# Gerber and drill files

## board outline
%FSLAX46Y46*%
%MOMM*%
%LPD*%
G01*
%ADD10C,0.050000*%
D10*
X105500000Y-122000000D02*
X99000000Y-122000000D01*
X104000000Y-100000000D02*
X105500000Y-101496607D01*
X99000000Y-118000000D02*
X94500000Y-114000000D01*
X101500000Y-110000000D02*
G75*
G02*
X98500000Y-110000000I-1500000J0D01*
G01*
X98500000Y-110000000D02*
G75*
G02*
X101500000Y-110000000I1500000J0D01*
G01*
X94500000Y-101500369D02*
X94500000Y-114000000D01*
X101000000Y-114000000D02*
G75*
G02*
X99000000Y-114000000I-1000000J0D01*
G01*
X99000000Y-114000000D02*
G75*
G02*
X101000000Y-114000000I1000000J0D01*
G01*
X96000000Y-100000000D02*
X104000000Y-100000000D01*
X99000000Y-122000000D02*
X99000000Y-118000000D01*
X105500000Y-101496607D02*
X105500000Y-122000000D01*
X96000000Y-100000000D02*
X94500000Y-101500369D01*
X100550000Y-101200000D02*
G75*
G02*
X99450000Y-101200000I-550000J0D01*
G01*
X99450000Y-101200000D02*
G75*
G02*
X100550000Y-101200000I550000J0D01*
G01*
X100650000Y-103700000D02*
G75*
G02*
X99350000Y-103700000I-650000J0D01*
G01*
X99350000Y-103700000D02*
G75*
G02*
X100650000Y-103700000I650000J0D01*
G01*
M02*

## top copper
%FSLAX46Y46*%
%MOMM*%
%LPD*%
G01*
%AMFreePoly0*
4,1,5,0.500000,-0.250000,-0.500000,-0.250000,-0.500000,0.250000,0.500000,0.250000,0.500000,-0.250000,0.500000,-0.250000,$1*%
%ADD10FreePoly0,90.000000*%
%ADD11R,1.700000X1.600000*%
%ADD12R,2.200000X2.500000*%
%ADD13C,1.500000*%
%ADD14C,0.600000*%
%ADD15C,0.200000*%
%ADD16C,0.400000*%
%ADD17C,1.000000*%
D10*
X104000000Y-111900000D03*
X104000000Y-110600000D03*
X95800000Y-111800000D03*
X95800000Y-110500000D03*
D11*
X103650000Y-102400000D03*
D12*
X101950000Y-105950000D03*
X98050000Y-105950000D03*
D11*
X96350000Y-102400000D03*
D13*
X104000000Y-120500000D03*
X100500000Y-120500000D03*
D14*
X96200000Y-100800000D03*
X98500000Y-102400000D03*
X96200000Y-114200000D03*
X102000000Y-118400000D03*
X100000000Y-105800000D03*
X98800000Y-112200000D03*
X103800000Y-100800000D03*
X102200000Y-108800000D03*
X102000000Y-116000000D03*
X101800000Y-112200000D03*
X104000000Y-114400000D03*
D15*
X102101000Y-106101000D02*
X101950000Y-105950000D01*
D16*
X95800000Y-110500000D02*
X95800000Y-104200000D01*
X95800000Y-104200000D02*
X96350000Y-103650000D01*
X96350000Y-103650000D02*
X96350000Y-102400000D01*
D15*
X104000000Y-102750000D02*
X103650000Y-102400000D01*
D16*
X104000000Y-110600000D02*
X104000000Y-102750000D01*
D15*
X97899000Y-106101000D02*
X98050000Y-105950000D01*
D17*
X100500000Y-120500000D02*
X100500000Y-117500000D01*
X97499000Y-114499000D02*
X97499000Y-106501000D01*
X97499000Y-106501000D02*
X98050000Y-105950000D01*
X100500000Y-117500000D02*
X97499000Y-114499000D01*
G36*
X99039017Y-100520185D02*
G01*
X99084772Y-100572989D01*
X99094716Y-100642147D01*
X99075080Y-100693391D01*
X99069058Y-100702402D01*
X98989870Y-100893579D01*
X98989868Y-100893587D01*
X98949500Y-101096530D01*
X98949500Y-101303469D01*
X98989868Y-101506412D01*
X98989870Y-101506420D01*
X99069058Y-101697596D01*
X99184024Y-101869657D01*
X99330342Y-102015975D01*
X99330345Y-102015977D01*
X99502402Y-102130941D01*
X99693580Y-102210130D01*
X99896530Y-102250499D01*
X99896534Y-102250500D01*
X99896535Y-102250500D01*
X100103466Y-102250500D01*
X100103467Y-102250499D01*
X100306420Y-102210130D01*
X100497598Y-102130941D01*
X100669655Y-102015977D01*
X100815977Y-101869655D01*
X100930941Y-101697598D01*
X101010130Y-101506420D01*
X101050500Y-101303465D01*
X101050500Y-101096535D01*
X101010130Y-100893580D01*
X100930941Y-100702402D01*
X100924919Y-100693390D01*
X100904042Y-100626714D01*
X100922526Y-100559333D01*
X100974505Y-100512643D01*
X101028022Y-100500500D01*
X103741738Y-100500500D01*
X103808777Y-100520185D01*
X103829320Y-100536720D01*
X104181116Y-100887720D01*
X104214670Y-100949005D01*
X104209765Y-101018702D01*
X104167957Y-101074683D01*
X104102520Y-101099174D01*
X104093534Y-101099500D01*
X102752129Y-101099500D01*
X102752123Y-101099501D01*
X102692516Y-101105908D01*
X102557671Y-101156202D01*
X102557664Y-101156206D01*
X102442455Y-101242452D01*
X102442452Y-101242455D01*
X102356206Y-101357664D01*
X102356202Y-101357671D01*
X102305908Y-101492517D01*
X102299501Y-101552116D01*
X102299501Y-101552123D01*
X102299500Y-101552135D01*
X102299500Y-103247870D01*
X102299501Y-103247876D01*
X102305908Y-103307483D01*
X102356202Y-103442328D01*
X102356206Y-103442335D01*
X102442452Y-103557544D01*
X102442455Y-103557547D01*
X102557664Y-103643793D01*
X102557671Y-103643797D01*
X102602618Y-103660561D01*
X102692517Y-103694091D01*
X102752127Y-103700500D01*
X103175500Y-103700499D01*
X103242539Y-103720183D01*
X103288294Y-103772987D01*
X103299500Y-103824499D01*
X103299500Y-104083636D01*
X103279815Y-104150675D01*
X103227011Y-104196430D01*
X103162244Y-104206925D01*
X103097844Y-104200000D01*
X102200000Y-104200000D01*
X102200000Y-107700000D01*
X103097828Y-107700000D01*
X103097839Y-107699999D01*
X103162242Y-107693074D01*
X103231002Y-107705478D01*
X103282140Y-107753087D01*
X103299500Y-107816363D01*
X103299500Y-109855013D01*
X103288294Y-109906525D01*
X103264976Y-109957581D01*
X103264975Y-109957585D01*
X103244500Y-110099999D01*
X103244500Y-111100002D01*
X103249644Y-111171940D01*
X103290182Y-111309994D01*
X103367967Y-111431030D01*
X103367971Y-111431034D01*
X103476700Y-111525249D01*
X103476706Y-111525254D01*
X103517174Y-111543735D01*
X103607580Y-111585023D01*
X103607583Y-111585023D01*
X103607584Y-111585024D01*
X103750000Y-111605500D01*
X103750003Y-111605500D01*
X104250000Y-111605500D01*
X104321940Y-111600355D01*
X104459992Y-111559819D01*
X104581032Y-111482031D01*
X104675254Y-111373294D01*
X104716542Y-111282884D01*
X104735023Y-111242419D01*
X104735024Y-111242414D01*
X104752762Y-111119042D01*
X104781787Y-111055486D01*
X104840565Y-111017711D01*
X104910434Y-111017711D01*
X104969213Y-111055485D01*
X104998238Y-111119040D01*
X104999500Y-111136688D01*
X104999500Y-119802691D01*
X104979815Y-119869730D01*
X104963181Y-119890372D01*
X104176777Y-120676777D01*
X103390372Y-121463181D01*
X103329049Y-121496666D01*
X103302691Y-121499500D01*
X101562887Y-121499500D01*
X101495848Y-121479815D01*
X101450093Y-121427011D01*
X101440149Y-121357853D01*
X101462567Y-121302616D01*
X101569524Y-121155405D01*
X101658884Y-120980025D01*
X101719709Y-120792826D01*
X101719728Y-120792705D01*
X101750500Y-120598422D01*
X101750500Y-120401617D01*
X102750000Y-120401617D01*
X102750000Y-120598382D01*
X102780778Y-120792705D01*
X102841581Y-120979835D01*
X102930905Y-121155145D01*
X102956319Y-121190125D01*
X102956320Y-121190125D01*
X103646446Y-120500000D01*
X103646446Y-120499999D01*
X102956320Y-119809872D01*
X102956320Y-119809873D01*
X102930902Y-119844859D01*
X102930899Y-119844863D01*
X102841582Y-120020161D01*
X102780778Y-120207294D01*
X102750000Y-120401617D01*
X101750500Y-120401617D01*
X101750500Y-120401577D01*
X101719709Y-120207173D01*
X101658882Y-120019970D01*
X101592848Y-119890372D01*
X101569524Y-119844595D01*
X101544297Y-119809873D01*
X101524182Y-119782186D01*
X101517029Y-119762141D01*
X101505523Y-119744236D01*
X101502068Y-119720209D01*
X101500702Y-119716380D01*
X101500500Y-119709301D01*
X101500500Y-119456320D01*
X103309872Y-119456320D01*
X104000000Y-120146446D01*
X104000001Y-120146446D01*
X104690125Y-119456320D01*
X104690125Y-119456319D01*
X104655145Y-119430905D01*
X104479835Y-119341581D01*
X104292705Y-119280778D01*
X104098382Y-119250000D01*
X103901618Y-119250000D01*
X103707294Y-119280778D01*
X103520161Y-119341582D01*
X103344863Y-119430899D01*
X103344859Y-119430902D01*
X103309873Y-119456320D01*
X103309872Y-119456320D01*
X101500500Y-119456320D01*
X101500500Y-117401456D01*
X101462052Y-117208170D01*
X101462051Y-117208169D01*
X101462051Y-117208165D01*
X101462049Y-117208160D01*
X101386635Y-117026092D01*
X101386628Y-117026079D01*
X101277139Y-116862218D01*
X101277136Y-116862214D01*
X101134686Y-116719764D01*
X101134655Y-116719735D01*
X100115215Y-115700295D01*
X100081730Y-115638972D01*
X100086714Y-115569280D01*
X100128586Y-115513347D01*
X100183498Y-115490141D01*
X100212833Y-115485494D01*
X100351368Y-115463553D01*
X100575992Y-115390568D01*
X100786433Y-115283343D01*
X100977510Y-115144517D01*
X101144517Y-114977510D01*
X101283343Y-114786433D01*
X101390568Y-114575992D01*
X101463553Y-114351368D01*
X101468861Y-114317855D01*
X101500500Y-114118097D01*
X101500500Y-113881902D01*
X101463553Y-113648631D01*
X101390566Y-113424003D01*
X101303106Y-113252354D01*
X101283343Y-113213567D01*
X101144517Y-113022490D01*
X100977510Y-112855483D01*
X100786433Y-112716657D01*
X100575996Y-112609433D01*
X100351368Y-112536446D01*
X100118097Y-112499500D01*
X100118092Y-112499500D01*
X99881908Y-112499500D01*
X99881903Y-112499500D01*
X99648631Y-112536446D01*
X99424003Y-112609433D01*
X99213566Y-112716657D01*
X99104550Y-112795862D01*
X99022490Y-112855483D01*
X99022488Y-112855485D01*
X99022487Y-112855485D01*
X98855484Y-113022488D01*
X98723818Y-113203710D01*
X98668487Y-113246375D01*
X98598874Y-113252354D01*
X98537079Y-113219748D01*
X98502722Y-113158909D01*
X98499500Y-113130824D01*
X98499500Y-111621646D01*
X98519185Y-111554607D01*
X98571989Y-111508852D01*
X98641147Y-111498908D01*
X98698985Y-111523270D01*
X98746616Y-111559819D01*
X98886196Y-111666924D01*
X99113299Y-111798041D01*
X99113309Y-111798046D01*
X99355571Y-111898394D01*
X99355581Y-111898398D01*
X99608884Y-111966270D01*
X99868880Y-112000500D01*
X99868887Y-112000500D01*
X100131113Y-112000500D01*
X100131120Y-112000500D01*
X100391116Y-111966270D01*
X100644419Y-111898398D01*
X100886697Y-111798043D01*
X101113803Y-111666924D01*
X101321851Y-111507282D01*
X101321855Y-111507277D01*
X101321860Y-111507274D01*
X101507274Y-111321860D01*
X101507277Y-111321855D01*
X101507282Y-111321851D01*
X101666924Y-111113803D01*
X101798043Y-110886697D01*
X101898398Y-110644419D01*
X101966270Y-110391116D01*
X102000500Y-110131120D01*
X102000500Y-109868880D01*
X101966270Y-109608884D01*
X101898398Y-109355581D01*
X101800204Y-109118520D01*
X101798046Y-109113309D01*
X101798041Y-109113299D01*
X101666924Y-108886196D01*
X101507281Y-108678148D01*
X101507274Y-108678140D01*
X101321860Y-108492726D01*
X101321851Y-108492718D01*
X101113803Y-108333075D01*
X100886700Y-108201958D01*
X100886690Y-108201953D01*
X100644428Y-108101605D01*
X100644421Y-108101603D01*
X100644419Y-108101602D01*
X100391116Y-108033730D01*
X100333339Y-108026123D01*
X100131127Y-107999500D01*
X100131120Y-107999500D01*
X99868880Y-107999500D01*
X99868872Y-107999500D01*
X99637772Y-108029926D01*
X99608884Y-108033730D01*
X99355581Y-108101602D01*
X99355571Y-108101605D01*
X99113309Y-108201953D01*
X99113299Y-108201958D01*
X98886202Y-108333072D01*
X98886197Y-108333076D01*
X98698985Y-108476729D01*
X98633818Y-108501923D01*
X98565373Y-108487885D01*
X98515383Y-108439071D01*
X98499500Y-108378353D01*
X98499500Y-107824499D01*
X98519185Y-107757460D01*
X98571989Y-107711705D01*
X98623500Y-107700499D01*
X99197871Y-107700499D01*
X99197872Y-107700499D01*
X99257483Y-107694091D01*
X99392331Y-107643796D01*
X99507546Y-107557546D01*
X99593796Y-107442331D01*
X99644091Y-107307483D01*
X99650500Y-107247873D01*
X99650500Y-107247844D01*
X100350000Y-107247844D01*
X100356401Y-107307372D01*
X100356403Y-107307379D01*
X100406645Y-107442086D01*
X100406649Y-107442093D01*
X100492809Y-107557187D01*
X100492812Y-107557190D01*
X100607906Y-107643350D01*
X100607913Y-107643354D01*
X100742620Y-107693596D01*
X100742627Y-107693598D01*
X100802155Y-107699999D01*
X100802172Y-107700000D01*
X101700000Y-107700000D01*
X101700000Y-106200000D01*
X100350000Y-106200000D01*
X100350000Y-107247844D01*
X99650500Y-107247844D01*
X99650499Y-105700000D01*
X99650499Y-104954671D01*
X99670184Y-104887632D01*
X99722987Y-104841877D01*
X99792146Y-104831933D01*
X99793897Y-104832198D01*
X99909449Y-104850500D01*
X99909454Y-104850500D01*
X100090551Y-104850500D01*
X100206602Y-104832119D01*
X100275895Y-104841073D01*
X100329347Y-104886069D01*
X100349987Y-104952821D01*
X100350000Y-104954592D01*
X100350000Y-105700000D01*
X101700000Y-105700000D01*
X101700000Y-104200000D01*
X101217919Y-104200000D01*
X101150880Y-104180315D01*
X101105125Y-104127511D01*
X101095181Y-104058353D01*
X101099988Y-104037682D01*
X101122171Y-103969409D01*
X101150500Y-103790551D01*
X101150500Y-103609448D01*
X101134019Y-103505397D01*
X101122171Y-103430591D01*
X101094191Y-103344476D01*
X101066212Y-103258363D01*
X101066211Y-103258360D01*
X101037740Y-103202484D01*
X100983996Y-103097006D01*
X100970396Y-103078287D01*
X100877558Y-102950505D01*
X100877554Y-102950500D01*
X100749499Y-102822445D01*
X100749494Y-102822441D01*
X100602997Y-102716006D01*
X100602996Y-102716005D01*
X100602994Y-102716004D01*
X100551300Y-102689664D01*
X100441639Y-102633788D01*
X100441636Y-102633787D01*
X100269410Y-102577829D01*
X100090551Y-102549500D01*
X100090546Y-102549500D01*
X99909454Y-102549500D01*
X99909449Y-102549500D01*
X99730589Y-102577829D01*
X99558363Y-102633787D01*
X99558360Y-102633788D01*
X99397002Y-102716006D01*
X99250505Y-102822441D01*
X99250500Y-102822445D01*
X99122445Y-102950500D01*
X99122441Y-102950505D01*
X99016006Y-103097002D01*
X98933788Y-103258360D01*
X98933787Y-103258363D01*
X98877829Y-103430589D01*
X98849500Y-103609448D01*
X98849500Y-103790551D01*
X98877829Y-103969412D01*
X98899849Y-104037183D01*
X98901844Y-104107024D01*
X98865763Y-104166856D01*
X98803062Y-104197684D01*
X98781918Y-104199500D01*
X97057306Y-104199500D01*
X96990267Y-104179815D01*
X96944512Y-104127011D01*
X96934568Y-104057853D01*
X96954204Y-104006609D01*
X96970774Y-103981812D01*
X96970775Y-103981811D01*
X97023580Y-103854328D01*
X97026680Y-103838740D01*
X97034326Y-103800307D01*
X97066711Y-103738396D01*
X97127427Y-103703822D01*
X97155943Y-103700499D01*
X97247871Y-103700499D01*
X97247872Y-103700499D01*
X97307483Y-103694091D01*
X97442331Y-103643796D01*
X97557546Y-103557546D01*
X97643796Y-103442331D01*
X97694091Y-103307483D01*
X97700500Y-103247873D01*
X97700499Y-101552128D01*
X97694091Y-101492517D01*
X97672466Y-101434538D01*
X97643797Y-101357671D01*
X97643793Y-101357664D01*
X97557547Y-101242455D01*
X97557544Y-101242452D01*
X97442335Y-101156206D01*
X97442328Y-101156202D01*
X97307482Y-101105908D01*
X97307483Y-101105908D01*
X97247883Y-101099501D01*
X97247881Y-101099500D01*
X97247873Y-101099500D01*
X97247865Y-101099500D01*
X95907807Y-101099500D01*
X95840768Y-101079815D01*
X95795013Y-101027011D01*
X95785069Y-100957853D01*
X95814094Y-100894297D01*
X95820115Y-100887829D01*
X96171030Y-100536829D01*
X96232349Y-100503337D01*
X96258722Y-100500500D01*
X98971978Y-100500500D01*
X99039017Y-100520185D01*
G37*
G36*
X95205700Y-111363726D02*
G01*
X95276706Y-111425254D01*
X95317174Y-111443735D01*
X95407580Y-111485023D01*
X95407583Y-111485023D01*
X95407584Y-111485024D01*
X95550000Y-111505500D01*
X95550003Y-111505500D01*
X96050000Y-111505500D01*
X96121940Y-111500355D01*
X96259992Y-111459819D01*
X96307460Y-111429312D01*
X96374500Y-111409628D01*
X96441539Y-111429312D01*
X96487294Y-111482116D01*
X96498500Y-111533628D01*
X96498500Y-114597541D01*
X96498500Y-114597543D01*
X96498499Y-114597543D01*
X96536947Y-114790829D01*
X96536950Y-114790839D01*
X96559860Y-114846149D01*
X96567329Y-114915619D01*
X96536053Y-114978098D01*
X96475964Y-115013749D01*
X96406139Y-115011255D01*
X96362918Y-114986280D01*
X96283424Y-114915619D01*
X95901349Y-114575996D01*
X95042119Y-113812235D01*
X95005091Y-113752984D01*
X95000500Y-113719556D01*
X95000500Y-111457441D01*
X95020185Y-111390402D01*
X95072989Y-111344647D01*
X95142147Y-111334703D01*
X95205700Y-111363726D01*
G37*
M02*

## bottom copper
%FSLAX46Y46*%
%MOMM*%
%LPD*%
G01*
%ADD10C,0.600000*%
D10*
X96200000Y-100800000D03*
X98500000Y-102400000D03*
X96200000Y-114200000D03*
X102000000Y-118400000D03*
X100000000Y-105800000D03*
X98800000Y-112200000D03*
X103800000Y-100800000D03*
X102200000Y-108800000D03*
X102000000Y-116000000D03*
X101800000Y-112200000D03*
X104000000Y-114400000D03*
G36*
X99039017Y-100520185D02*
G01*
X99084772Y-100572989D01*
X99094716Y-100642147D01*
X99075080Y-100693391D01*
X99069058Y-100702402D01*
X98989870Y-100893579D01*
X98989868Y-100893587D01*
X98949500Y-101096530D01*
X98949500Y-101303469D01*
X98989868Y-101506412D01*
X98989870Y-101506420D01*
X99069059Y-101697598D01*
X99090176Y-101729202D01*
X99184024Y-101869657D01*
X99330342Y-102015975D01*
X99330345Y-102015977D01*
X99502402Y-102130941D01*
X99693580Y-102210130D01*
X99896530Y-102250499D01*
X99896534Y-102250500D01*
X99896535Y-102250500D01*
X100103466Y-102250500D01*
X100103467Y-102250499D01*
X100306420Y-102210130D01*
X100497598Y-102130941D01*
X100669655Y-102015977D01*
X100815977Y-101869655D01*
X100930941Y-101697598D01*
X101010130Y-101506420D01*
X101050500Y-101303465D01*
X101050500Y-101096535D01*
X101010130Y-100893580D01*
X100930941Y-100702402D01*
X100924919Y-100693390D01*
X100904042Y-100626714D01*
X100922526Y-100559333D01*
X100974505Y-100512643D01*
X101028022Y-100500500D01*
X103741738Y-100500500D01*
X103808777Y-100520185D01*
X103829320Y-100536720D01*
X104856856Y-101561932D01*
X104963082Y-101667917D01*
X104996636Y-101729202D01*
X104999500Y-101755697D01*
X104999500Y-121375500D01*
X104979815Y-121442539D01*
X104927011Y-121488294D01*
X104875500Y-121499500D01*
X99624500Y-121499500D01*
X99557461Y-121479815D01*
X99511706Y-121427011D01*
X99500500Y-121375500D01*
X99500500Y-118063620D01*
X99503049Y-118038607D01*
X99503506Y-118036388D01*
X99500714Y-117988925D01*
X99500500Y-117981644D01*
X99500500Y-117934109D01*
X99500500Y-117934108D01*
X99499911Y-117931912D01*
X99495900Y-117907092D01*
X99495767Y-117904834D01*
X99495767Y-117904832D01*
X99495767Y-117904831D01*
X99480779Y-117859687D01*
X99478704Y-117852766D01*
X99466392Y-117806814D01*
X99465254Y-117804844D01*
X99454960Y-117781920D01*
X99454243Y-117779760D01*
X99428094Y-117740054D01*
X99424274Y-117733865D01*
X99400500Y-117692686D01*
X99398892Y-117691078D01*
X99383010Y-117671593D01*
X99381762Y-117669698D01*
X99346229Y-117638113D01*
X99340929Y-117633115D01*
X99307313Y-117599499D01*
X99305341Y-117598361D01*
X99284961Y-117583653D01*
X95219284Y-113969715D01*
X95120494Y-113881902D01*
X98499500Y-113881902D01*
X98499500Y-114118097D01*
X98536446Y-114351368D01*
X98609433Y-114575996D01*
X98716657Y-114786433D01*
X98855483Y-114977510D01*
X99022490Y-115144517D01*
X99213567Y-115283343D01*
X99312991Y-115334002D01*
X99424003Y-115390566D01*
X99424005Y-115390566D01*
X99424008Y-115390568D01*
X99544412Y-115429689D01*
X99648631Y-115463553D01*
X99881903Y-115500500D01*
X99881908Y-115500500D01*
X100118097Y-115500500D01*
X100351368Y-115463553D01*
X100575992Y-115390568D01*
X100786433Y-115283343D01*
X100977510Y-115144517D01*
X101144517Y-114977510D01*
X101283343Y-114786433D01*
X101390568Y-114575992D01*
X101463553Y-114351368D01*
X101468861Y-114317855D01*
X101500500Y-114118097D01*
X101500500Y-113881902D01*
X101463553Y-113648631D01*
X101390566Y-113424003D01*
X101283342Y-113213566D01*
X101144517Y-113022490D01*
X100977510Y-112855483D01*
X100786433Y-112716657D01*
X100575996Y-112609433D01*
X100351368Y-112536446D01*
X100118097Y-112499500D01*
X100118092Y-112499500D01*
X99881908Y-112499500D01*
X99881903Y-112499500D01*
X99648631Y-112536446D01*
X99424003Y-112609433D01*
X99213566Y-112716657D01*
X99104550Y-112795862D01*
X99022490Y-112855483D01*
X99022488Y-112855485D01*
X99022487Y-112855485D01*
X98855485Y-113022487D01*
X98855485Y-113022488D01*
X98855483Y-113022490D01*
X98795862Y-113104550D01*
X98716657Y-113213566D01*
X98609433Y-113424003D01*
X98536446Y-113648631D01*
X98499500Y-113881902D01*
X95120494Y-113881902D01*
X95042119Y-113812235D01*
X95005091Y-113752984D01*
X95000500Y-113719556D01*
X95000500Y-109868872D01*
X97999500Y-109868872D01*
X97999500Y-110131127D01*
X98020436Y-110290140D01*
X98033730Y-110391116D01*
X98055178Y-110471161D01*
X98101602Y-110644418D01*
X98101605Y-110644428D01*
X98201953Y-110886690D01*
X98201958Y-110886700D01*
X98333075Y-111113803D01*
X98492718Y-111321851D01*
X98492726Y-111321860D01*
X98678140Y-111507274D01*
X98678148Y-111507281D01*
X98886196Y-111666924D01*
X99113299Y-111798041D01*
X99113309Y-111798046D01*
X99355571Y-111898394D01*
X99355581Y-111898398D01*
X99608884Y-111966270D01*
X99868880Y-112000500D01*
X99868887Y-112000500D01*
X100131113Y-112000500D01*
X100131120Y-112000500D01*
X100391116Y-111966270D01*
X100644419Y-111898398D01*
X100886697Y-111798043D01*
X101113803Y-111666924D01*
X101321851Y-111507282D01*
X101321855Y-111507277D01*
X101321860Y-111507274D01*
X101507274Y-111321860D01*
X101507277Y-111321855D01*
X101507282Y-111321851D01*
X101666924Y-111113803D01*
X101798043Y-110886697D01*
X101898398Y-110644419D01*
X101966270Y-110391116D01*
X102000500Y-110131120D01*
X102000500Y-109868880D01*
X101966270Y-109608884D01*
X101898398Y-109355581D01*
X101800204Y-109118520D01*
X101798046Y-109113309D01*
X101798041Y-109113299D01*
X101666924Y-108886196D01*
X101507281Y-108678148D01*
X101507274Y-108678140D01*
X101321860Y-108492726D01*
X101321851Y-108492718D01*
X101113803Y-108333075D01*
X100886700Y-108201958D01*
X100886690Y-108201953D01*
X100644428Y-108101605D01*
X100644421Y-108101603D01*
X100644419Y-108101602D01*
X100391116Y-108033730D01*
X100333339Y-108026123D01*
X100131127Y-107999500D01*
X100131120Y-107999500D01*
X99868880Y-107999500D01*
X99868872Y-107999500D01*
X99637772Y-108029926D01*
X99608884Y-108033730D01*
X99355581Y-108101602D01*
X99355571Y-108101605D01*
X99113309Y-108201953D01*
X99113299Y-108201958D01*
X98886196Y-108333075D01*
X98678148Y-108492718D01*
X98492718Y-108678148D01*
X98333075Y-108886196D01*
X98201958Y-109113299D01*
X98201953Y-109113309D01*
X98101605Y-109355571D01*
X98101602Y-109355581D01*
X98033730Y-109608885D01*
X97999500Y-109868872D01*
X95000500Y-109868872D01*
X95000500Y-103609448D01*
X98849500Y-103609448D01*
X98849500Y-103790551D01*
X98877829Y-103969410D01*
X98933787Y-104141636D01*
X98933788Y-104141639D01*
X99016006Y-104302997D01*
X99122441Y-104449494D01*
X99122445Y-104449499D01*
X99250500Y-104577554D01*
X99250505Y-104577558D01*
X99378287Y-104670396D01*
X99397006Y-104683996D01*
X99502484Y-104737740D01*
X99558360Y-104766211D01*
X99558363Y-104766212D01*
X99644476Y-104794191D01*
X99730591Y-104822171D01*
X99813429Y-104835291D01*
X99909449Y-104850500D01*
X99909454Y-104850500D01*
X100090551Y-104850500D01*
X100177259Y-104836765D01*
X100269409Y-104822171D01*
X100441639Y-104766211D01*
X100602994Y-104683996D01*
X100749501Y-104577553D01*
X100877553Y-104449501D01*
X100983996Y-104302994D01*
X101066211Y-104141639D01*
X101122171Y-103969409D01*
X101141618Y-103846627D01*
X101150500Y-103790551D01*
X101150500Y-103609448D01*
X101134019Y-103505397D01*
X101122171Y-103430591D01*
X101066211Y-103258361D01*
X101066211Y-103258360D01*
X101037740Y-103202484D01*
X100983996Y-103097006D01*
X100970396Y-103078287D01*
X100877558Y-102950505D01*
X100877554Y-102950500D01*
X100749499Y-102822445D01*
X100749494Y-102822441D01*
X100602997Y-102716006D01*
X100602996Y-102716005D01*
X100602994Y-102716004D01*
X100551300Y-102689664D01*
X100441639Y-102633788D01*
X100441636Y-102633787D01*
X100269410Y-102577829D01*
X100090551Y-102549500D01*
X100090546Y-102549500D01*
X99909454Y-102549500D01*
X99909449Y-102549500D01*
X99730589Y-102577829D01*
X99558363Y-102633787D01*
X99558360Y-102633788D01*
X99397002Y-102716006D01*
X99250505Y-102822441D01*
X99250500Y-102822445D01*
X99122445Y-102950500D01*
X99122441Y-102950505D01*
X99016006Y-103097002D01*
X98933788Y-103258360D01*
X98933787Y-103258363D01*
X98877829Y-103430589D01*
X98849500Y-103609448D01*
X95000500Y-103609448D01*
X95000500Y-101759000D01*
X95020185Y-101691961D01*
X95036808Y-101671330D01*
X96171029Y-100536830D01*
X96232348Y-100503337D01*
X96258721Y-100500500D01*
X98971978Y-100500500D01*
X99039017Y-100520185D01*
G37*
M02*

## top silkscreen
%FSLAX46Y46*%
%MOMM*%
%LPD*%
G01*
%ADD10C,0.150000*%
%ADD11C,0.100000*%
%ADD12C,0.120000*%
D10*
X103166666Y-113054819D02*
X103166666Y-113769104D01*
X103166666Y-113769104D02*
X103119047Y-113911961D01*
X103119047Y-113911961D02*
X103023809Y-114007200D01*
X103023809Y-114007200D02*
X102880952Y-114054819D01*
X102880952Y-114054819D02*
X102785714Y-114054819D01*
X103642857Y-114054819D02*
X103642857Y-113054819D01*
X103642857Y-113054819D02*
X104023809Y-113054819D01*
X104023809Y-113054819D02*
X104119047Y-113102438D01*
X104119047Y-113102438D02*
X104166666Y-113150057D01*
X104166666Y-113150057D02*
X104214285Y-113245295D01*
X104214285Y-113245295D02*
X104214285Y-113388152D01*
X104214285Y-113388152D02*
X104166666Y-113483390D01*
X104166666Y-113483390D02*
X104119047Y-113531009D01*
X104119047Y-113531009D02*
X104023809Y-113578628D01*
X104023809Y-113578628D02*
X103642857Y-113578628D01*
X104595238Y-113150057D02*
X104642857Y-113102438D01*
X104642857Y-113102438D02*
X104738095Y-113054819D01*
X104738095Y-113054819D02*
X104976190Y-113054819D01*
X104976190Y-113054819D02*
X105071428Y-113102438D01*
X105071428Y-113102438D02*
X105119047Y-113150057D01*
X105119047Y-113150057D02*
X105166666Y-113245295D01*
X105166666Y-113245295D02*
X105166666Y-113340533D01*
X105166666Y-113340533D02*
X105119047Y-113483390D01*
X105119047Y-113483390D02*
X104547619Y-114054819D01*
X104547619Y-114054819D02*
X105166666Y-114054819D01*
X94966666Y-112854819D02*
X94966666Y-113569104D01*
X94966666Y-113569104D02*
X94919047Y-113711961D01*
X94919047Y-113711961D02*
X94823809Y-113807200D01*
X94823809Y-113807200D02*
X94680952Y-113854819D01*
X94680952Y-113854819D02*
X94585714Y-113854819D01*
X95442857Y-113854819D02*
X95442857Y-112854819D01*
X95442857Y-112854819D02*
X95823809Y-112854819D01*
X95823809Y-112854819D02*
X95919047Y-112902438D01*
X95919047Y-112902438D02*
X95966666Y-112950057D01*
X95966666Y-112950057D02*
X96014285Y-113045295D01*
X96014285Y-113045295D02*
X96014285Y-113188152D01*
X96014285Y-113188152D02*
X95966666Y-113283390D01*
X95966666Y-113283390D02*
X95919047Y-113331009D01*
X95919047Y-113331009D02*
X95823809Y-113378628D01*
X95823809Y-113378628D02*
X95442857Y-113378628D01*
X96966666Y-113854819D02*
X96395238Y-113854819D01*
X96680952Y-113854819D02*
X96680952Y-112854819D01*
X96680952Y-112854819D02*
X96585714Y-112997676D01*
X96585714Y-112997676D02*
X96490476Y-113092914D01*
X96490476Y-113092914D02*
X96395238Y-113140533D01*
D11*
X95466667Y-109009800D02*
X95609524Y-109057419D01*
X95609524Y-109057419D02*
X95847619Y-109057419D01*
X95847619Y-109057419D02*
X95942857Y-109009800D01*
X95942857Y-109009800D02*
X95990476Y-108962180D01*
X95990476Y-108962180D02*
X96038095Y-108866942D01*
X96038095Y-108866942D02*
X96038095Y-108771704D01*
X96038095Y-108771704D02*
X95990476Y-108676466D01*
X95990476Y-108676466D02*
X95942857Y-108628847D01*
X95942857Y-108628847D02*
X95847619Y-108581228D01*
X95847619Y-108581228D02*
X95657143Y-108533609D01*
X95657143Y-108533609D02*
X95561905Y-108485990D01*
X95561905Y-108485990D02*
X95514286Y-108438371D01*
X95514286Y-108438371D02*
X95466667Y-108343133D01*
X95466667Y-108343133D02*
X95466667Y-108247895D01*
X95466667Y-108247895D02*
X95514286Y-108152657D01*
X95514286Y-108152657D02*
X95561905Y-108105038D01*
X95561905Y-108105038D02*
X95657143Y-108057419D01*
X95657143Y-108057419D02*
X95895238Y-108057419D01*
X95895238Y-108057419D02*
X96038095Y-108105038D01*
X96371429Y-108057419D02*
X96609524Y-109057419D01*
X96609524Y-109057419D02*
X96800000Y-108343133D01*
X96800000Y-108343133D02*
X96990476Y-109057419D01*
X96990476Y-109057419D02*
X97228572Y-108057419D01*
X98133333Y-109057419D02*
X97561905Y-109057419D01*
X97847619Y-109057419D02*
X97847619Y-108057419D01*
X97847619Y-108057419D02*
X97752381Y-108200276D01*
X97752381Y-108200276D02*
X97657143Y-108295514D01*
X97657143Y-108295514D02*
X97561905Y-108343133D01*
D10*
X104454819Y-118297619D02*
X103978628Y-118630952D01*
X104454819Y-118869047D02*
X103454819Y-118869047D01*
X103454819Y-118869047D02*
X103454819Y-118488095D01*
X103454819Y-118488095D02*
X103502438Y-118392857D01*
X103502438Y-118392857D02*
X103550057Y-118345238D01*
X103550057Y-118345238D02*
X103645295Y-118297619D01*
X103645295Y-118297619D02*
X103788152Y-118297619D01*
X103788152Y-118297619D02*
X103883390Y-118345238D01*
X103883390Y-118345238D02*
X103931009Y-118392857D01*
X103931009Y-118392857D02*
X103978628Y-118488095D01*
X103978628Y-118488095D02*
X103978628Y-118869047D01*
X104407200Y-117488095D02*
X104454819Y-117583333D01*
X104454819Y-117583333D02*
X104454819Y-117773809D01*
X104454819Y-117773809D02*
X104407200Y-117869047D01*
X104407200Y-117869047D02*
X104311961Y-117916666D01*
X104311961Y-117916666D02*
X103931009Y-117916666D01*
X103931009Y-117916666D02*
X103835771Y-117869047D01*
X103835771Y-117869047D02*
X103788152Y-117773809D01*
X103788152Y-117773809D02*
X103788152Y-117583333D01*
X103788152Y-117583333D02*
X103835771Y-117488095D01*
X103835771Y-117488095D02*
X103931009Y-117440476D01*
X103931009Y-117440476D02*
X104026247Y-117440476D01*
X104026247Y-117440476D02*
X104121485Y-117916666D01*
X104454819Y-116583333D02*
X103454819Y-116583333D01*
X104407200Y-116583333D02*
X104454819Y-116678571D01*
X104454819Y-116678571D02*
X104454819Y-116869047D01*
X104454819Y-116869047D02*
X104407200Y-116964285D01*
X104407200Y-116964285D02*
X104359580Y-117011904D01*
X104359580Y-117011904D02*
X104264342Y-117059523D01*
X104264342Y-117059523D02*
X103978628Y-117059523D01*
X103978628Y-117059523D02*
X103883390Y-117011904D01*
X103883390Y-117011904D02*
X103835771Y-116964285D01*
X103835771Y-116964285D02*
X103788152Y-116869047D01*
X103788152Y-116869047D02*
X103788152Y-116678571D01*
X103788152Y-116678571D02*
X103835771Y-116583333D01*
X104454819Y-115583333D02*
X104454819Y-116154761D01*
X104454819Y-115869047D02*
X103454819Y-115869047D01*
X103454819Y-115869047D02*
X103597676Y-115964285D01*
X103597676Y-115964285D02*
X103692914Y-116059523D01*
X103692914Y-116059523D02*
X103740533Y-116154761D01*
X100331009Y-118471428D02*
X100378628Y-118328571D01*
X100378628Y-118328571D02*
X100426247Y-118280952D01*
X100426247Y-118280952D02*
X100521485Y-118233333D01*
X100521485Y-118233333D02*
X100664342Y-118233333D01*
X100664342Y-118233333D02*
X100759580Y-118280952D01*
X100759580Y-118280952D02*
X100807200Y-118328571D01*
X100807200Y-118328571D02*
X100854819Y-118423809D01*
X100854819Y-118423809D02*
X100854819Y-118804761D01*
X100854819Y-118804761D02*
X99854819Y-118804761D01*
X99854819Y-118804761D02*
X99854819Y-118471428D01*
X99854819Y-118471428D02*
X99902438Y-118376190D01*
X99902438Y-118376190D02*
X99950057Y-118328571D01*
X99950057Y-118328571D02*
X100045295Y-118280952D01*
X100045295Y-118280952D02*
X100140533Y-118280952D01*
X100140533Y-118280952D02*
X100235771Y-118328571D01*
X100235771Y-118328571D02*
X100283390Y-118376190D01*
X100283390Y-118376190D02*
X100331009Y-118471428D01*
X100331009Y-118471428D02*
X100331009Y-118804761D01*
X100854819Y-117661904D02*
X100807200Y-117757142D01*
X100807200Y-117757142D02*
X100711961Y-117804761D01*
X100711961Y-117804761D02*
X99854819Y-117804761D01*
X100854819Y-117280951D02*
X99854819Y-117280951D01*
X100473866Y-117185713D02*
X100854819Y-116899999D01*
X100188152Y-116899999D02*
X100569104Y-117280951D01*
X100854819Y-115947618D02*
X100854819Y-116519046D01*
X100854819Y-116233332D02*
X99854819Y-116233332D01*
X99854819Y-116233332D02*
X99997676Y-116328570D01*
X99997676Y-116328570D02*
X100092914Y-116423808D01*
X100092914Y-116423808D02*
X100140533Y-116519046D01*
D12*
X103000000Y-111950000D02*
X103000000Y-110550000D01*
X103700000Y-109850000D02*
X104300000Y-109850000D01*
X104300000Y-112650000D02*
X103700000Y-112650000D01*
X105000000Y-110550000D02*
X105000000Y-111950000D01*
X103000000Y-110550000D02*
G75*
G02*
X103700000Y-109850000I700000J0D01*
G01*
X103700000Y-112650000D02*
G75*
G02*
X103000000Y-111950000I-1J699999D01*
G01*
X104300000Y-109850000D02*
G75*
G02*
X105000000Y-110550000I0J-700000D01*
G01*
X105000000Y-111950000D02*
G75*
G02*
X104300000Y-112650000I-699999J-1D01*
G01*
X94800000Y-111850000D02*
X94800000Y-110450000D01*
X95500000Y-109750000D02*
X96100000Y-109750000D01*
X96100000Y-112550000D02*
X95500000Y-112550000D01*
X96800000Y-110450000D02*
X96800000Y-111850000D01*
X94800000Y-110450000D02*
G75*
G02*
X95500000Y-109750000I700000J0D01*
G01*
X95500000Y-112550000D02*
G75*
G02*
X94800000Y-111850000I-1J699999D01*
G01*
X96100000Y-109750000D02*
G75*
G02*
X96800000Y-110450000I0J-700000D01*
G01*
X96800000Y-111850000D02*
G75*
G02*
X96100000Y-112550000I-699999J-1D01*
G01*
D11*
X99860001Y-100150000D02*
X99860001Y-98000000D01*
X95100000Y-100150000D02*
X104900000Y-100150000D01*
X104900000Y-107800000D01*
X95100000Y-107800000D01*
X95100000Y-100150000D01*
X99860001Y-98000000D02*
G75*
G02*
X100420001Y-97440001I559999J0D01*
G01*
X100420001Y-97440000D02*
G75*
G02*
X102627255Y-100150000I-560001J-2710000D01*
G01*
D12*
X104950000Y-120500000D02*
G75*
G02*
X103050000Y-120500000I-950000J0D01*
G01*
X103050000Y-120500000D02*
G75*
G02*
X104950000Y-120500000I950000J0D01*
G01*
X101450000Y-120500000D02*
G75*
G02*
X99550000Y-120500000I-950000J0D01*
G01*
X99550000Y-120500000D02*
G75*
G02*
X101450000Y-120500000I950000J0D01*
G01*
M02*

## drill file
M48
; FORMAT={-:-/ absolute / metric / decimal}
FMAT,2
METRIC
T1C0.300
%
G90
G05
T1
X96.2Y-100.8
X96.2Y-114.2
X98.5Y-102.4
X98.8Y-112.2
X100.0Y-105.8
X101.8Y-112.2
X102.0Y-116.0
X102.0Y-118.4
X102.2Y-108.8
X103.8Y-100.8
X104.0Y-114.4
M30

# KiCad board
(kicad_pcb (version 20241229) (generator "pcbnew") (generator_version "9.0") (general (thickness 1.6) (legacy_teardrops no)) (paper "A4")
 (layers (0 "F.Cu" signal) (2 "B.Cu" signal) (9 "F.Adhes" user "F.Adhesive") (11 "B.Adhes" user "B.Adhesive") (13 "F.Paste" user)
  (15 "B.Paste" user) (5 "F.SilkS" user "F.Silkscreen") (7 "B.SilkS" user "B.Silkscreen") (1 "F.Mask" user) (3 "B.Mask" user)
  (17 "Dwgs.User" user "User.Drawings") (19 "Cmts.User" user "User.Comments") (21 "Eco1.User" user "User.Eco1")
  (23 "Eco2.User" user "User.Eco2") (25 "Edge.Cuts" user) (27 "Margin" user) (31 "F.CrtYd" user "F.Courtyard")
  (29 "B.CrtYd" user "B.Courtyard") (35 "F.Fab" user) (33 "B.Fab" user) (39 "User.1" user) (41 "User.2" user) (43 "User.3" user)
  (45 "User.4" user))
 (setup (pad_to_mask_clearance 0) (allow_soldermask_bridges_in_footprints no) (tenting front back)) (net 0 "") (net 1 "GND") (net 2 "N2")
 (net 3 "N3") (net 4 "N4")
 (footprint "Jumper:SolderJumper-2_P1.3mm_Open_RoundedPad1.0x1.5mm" (layer "F.Cu") (at 104 111.25 90)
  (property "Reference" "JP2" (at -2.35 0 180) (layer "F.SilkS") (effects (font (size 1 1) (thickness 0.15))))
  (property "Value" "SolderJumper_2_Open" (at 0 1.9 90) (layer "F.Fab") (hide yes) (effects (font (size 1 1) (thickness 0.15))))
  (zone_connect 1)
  (fp_line (start -0.7 -1) (end 0.7 -1) (stroke (width 0.12) (type solid)) (layer "F.SilkS"))
  (fp_line (start 1.4 -0.3) (end 1.4 0.3) (stroke (width 0.12) (type solid)) (layer "F.SilkS"))
  (fp_line (start -1.4 0.3) (end -1.4 -0.3) (stroke (width 0.12) (type solid)) (layer "F.SilkS"))
  (fp_line (start 0.7 1) (end -0.7 1) (stroke (width 0.12) (type solid)) (layer "F.SilkS"))
  (fp_arc (start 0.7 -1) (mid 1.194975 -0.794975) (end 1.4 -0.3) (stroke (width 0.12) (type solid)) (layer "F.SilkS"))
  (fp_arc (start -1.4 -0.3) (mid -1.194975 -0.794975) (end -0.7 -1) (stroke (width 0.12) (type solid)) (layer "F.SilkS"))
  (fp_arc (start 1.4 0.3) (mid 1.194975 0.794975) (end 0.7 1) (stroke (width 0.12) (type solid)) (layer "F.SilkS"))
  (fp_arc (start -0.7 1) (mid -1.194975 0.794975) (end -1.4 0.3) (stroke (width 0.12) (type solid)) (layer "F.SilkS"))
  (pad "1" smd custom (at -0.65 0 90) (size 1 0.5) (layers "F.Cu" "F.Mask") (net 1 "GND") (zone_connect 2) (thermal_bridge_angle 45)
   (options (clearance outline) (anchor rect)) (primitives))
  (pad "2" smd custom (at 0.65 0 90) (size 1 0.5) (layers "F.Cu" "F.Mask") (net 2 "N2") (zone_connect 2) (thermal_bridge_angle 45)
   (options (clearance outline) (anchor rect)) (primitives)))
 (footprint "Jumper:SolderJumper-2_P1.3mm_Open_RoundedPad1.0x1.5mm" (layer "F.Cu") (at 95.8 111.15 90)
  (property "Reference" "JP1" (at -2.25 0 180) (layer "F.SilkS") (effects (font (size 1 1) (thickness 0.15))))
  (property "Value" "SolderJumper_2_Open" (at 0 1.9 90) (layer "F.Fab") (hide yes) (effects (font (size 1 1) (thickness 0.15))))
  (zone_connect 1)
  (fp_line (start -0.7 -1) (end 0.7 -1) (stroke (width 0.12) (type solid)) (layer "F.SilkS"))
  (fp_line (start 1.4 -0.3) (end 1.4 0.3) (stroke (width 0.12) (type solid)) (layer "F.SilkS"))
  (fp_line (start -1.4 0.3) (end -1.4 -0.3) (stroke (width 0.12) (type solid)) (layer "F.SilkS"))
  (fp_line (start 0.7 1) (end -0.7 1) (stroke (width 0.12) (type solid)) (layer "F.SilkS"))
  (fp_arc (start 0.7 -1) (mid 1.194975 -0.794975) (end 1.4 -0.3) (stroke (width 0.12) (type solid)) (layer "F.SilkS"))
  (fp_arc (start -1.4 -0.3) (mid -1.194975 -0.794975) (end -0.7 -1) (stroke (width 0.12) (type solid)) (layer "F.SilkS"))
  (fp_arc (start 1.4 0.3) (mid 1.194975 0.794975) (end 0.7 1) (stroke (width 0.12) (type solid)) (layer "F.SilkS"))
  (fp_arc (start -0.7 1) (mid -1.194975 0.794975) (end -1.4 0.3) (stroke (width 0.12) (type solid)) (layer "F.SilkS"))
  (pad "1" smd custom (at -0.65 0 90) (size 1 0.5) (layers "F.Cu" "F.Mask") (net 1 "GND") (zone_connect 2) (thermal_bridge_angle 45)
   (options (clearance outline) (anchor rect)) (primitives))
  (pad "2" smd custom (at 0.65 0 90) (size 1 0.5) (layers "F.Cu" "F.Mask") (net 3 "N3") (zone_connect 2) (thermal_bridge_angle 45)
   (options (clearance outline) (anchor rect)) (primitives)))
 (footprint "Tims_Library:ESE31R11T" (layer "F.Cu") (at 100 101.2)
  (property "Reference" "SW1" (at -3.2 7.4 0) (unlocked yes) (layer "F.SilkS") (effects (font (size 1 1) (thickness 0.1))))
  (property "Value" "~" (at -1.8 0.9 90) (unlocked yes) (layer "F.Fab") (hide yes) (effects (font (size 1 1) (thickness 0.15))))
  (fp_line (start -0.139999 -1.05) (end -0.139999 -3.2) (stroke (width 0.1) (type default)) (layer "F.SilkS"))
  (fp_rect (start -4.9 -1.05) (end 4.9 6.6) (stroke (width 0.1) (type default)) (fill no) (layer "F.SilkS"))
  (fp_arc (start -0.139999 -3.2) (mid 0.024021 -3.59598) (end 0.420001 -3.76) (stroke (width 0.1) (type default)) (layer "F.SilkS"))
  (fp_arc (start 0.420001 -3.76) (mid 2.00562 -2.797575) (end 2.627256 -1.05) (stroke (width 0.1) (type default)) (layer "F.SilkS"))
  (fp_circle (center 0 0) (end 0 -0.55) (stroke (width 0.05) (type default)) (fill no) (layer "Edge.Cuts"))
  (fp_circle (center 0 2.5) (end 0 1.85) (stroke (width 0.05) (type default)) (fill no) (layer "Edge.Cuts"))
  (pad "1" smd rect (at 3.65 1.2) (size 1.7 1.6) (layers "F.Cu" "F.Mask" "F.Paste") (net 2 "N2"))
  (pad "2" smd rect (at 1.95 4.75) (size 2.2 2.5) (layers "F.Cu" "F.Mask" "F.Paste") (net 1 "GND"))
  (pad "3" smd rect (at -1.95 4.75) (size 2.2 2.5) (layers "F.Cu" "F.Mask" "F.Paste") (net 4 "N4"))
  (pad "4" smd rect (at -3.65 1.2) (size 1.7 1.6) (layers "F.Cu" "F.Mask" "F.Paste") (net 3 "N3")))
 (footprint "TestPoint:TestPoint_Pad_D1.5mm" (layer "F.Cu") (at 104 120.5 -90)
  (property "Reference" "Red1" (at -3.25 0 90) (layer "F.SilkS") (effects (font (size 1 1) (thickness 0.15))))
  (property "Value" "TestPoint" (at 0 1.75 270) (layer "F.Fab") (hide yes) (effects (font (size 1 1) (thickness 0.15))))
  (fp_circle (center 0 0) (end 0 0.95) (stroke (width 0.12) (type solid)) (fill no) (layer "F.SilkS"))
  (pad "1" smd circle (at 0 0 270) (size 1.5 1.5) (layers "F.Cu" "F.Mask") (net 1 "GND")))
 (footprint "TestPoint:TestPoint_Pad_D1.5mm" (layer "F.Cu") (at 100.5 120.5 -90)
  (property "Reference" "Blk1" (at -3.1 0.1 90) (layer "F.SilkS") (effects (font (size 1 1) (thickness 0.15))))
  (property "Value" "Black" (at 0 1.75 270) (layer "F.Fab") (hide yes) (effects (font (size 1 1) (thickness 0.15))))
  (fp_circle (center 0 0) (end 0 0.95) (stroke (width 0.12) (type solid)) (fill no) (layer "F.SilkS"))
  (pad "1" smd circle (at 0 0 270) (size 1.5 1.5) (layers "F.Cu" "F.Mask") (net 4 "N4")))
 (gr_line (start 105.5 122) (end 99 122) (stroke (width 0.05) (type default)) (layer "Edge.Cuts"))
 (gr_line (start 104 100) (end 105.5 101.496607) (stroke (width 0.05) (type default)) (layer "Edge.Cuts"))
 (gr_line (start 99 118) (end 94.5 114) (stroke (width 0.05) (type default)) (layer "Edge.Cuts"))
 (gr_circle (center 100 110) (end 98.5 110) (stroke (width 0.05) (type default)) (fill no) (layer "Edge.Cuts"))
 (gr_line (start 94.5 101.500369) (end 94.5 114) (stroke (width 0.05) (type default)) (layer "Edge.Cuts"))
 (gr_circle (center 100 114) (end 100 115) (stroke (width 0.05) (type default)) (fill no) (layer "Edge.Cuts"))
 (gr_line (start 96 100) (end 104 100) (stroke (width 0.05) (type default)) (layer "Edge.Cuts"))
 (gr_line (start 99 122) (end 99 118) (stroke (width 0.05) (type default)) (layer "Edge.Cuts"))
 (gr_line (start 105.5 101.496607) (end 105.5 122) (stroke (width 0.05) (type default)) (layer "Edge.Cuts"))
 (gr_line (start 96 100) (end 94.5 101.500369) (stroke (width 0.05) (type default)) (layer "Edge.Cuts"))
 (segment (start 102.101 106.101) (end 101.95 105.95) (width 0.2) (layer "F.Cu") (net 1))
 (via (at 96.2 100.8) (size 0.6) (drill 0.3) (layers "F.Cu" "B.Cu") (free yes) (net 1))
 (via (at 98.5 102.4) (size 0.6) (drill 0.3) (layers "F.Cu" "B.Cu") (free yes) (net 1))
 (via (at 96.2 114.2) (size 0.6) (drill 0.3) (layers "F.Cu" "B.Cu") (free yes) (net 1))
 (via (at 102 118.4) (size 0.6) (drill 0.3) (layers "F.Cu" "B.Cu") (free yes) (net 1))
 (via (at 100 105.8) (size 0.6) (drill 0.3) (layers "F.Cu" "B.Cu") (free yes) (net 1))
 (via (at 98.8 112.2) (size 0.6) (drill 0.3) (layers "F.Cu" "B.Cu") (free yes) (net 1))
 (via (at 103.8 100.8) (size 0.6) (drill 0.3) (layers "F.Cu" "B.Cu") (free yes) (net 1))
 (via (at 102.2 108.8) (size 0.6) (drill 0.3) (layers "F.Cu" "B.Cu") (free yes) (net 1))
 (via (at 102 116) (size 0.6) (drill 0.3) (layers "F.Cu" "B.Cu") (free yes) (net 1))
 (via (at 101.8 112.2) (size 0.6) (drill 0.3) (layers "F.Cu" "B.Cu") (free yes) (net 1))
 (via (at 104 114.4) (size 0.6) (drill 0.3) (layers "F.Cu" "B.Cu") (free yes) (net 1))
 (segment (start 95.8 110.5) (end 95.8 104.2) (width 0.4) (layer "F.Cu") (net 3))
 (segment (start 95.8 104.2) (end 96.35 103.65) (width 0.4) (layer "F.Cu") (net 3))
 (segment (start 96.35 103.65) (end 96.35 102.4) (width 0.4) (layer "F.Cu") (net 3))
 (segment (start 104 102.75) (end 103.65 102.4) (width 0.2) (layer "F.Cu") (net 2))
 (segment (start 104 110.6) (end 104 102.75) (width 0.4) (layer "F.Cu") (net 2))
 (segment (start 97.899 106.101) (end 98.05 105.95) (width 0.2) (layer "F.Cu") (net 4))
 (segment (start 100.5 120.5) (end 100.5 117.5) (width 1) (layer "F.Cu") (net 4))
 (segment (start 97.499 114.499) (end 97.499 106.501) (width 1) (layer "F.Cu") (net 4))
 (segment (start 97.499 106.501) (end 98.05 105.95) (width 1) (layer "F.Cu") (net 4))
 (segment (start 100.5 117.5) (end 97.499 114.499) (width 1) (layer "F.Cu") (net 4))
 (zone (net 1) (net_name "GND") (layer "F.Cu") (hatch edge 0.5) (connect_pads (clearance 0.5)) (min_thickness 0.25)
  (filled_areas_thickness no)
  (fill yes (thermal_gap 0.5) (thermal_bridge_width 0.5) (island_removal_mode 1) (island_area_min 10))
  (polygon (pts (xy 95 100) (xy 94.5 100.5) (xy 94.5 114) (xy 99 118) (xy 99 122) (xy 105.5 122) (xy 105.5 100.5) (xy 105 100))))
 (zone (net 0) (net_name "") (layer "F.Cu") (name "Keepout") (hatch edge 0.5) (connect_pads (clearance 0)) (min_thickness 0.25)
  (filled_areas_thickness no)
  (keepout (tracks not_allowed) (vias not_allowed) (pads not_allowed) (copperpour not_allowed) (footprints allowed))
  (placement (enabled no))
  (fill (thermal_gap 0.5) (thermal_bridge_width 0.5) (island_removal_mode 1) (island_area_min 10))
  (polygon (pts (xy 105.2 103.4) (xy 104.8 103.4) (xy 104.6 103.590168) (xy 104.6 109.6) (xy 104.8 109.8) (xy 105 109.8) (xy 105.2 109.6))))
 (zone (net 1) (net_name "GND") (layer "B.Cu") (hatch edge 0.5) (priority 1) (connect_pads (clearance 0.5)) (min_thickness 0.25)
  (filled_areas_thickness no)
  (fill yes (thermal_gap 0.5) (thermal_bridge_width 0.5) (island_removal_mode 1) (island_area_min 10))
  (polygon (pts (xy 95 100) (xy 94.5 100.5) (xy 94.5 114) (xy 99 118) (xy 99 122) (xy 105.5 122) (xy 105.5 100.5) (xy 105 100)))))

